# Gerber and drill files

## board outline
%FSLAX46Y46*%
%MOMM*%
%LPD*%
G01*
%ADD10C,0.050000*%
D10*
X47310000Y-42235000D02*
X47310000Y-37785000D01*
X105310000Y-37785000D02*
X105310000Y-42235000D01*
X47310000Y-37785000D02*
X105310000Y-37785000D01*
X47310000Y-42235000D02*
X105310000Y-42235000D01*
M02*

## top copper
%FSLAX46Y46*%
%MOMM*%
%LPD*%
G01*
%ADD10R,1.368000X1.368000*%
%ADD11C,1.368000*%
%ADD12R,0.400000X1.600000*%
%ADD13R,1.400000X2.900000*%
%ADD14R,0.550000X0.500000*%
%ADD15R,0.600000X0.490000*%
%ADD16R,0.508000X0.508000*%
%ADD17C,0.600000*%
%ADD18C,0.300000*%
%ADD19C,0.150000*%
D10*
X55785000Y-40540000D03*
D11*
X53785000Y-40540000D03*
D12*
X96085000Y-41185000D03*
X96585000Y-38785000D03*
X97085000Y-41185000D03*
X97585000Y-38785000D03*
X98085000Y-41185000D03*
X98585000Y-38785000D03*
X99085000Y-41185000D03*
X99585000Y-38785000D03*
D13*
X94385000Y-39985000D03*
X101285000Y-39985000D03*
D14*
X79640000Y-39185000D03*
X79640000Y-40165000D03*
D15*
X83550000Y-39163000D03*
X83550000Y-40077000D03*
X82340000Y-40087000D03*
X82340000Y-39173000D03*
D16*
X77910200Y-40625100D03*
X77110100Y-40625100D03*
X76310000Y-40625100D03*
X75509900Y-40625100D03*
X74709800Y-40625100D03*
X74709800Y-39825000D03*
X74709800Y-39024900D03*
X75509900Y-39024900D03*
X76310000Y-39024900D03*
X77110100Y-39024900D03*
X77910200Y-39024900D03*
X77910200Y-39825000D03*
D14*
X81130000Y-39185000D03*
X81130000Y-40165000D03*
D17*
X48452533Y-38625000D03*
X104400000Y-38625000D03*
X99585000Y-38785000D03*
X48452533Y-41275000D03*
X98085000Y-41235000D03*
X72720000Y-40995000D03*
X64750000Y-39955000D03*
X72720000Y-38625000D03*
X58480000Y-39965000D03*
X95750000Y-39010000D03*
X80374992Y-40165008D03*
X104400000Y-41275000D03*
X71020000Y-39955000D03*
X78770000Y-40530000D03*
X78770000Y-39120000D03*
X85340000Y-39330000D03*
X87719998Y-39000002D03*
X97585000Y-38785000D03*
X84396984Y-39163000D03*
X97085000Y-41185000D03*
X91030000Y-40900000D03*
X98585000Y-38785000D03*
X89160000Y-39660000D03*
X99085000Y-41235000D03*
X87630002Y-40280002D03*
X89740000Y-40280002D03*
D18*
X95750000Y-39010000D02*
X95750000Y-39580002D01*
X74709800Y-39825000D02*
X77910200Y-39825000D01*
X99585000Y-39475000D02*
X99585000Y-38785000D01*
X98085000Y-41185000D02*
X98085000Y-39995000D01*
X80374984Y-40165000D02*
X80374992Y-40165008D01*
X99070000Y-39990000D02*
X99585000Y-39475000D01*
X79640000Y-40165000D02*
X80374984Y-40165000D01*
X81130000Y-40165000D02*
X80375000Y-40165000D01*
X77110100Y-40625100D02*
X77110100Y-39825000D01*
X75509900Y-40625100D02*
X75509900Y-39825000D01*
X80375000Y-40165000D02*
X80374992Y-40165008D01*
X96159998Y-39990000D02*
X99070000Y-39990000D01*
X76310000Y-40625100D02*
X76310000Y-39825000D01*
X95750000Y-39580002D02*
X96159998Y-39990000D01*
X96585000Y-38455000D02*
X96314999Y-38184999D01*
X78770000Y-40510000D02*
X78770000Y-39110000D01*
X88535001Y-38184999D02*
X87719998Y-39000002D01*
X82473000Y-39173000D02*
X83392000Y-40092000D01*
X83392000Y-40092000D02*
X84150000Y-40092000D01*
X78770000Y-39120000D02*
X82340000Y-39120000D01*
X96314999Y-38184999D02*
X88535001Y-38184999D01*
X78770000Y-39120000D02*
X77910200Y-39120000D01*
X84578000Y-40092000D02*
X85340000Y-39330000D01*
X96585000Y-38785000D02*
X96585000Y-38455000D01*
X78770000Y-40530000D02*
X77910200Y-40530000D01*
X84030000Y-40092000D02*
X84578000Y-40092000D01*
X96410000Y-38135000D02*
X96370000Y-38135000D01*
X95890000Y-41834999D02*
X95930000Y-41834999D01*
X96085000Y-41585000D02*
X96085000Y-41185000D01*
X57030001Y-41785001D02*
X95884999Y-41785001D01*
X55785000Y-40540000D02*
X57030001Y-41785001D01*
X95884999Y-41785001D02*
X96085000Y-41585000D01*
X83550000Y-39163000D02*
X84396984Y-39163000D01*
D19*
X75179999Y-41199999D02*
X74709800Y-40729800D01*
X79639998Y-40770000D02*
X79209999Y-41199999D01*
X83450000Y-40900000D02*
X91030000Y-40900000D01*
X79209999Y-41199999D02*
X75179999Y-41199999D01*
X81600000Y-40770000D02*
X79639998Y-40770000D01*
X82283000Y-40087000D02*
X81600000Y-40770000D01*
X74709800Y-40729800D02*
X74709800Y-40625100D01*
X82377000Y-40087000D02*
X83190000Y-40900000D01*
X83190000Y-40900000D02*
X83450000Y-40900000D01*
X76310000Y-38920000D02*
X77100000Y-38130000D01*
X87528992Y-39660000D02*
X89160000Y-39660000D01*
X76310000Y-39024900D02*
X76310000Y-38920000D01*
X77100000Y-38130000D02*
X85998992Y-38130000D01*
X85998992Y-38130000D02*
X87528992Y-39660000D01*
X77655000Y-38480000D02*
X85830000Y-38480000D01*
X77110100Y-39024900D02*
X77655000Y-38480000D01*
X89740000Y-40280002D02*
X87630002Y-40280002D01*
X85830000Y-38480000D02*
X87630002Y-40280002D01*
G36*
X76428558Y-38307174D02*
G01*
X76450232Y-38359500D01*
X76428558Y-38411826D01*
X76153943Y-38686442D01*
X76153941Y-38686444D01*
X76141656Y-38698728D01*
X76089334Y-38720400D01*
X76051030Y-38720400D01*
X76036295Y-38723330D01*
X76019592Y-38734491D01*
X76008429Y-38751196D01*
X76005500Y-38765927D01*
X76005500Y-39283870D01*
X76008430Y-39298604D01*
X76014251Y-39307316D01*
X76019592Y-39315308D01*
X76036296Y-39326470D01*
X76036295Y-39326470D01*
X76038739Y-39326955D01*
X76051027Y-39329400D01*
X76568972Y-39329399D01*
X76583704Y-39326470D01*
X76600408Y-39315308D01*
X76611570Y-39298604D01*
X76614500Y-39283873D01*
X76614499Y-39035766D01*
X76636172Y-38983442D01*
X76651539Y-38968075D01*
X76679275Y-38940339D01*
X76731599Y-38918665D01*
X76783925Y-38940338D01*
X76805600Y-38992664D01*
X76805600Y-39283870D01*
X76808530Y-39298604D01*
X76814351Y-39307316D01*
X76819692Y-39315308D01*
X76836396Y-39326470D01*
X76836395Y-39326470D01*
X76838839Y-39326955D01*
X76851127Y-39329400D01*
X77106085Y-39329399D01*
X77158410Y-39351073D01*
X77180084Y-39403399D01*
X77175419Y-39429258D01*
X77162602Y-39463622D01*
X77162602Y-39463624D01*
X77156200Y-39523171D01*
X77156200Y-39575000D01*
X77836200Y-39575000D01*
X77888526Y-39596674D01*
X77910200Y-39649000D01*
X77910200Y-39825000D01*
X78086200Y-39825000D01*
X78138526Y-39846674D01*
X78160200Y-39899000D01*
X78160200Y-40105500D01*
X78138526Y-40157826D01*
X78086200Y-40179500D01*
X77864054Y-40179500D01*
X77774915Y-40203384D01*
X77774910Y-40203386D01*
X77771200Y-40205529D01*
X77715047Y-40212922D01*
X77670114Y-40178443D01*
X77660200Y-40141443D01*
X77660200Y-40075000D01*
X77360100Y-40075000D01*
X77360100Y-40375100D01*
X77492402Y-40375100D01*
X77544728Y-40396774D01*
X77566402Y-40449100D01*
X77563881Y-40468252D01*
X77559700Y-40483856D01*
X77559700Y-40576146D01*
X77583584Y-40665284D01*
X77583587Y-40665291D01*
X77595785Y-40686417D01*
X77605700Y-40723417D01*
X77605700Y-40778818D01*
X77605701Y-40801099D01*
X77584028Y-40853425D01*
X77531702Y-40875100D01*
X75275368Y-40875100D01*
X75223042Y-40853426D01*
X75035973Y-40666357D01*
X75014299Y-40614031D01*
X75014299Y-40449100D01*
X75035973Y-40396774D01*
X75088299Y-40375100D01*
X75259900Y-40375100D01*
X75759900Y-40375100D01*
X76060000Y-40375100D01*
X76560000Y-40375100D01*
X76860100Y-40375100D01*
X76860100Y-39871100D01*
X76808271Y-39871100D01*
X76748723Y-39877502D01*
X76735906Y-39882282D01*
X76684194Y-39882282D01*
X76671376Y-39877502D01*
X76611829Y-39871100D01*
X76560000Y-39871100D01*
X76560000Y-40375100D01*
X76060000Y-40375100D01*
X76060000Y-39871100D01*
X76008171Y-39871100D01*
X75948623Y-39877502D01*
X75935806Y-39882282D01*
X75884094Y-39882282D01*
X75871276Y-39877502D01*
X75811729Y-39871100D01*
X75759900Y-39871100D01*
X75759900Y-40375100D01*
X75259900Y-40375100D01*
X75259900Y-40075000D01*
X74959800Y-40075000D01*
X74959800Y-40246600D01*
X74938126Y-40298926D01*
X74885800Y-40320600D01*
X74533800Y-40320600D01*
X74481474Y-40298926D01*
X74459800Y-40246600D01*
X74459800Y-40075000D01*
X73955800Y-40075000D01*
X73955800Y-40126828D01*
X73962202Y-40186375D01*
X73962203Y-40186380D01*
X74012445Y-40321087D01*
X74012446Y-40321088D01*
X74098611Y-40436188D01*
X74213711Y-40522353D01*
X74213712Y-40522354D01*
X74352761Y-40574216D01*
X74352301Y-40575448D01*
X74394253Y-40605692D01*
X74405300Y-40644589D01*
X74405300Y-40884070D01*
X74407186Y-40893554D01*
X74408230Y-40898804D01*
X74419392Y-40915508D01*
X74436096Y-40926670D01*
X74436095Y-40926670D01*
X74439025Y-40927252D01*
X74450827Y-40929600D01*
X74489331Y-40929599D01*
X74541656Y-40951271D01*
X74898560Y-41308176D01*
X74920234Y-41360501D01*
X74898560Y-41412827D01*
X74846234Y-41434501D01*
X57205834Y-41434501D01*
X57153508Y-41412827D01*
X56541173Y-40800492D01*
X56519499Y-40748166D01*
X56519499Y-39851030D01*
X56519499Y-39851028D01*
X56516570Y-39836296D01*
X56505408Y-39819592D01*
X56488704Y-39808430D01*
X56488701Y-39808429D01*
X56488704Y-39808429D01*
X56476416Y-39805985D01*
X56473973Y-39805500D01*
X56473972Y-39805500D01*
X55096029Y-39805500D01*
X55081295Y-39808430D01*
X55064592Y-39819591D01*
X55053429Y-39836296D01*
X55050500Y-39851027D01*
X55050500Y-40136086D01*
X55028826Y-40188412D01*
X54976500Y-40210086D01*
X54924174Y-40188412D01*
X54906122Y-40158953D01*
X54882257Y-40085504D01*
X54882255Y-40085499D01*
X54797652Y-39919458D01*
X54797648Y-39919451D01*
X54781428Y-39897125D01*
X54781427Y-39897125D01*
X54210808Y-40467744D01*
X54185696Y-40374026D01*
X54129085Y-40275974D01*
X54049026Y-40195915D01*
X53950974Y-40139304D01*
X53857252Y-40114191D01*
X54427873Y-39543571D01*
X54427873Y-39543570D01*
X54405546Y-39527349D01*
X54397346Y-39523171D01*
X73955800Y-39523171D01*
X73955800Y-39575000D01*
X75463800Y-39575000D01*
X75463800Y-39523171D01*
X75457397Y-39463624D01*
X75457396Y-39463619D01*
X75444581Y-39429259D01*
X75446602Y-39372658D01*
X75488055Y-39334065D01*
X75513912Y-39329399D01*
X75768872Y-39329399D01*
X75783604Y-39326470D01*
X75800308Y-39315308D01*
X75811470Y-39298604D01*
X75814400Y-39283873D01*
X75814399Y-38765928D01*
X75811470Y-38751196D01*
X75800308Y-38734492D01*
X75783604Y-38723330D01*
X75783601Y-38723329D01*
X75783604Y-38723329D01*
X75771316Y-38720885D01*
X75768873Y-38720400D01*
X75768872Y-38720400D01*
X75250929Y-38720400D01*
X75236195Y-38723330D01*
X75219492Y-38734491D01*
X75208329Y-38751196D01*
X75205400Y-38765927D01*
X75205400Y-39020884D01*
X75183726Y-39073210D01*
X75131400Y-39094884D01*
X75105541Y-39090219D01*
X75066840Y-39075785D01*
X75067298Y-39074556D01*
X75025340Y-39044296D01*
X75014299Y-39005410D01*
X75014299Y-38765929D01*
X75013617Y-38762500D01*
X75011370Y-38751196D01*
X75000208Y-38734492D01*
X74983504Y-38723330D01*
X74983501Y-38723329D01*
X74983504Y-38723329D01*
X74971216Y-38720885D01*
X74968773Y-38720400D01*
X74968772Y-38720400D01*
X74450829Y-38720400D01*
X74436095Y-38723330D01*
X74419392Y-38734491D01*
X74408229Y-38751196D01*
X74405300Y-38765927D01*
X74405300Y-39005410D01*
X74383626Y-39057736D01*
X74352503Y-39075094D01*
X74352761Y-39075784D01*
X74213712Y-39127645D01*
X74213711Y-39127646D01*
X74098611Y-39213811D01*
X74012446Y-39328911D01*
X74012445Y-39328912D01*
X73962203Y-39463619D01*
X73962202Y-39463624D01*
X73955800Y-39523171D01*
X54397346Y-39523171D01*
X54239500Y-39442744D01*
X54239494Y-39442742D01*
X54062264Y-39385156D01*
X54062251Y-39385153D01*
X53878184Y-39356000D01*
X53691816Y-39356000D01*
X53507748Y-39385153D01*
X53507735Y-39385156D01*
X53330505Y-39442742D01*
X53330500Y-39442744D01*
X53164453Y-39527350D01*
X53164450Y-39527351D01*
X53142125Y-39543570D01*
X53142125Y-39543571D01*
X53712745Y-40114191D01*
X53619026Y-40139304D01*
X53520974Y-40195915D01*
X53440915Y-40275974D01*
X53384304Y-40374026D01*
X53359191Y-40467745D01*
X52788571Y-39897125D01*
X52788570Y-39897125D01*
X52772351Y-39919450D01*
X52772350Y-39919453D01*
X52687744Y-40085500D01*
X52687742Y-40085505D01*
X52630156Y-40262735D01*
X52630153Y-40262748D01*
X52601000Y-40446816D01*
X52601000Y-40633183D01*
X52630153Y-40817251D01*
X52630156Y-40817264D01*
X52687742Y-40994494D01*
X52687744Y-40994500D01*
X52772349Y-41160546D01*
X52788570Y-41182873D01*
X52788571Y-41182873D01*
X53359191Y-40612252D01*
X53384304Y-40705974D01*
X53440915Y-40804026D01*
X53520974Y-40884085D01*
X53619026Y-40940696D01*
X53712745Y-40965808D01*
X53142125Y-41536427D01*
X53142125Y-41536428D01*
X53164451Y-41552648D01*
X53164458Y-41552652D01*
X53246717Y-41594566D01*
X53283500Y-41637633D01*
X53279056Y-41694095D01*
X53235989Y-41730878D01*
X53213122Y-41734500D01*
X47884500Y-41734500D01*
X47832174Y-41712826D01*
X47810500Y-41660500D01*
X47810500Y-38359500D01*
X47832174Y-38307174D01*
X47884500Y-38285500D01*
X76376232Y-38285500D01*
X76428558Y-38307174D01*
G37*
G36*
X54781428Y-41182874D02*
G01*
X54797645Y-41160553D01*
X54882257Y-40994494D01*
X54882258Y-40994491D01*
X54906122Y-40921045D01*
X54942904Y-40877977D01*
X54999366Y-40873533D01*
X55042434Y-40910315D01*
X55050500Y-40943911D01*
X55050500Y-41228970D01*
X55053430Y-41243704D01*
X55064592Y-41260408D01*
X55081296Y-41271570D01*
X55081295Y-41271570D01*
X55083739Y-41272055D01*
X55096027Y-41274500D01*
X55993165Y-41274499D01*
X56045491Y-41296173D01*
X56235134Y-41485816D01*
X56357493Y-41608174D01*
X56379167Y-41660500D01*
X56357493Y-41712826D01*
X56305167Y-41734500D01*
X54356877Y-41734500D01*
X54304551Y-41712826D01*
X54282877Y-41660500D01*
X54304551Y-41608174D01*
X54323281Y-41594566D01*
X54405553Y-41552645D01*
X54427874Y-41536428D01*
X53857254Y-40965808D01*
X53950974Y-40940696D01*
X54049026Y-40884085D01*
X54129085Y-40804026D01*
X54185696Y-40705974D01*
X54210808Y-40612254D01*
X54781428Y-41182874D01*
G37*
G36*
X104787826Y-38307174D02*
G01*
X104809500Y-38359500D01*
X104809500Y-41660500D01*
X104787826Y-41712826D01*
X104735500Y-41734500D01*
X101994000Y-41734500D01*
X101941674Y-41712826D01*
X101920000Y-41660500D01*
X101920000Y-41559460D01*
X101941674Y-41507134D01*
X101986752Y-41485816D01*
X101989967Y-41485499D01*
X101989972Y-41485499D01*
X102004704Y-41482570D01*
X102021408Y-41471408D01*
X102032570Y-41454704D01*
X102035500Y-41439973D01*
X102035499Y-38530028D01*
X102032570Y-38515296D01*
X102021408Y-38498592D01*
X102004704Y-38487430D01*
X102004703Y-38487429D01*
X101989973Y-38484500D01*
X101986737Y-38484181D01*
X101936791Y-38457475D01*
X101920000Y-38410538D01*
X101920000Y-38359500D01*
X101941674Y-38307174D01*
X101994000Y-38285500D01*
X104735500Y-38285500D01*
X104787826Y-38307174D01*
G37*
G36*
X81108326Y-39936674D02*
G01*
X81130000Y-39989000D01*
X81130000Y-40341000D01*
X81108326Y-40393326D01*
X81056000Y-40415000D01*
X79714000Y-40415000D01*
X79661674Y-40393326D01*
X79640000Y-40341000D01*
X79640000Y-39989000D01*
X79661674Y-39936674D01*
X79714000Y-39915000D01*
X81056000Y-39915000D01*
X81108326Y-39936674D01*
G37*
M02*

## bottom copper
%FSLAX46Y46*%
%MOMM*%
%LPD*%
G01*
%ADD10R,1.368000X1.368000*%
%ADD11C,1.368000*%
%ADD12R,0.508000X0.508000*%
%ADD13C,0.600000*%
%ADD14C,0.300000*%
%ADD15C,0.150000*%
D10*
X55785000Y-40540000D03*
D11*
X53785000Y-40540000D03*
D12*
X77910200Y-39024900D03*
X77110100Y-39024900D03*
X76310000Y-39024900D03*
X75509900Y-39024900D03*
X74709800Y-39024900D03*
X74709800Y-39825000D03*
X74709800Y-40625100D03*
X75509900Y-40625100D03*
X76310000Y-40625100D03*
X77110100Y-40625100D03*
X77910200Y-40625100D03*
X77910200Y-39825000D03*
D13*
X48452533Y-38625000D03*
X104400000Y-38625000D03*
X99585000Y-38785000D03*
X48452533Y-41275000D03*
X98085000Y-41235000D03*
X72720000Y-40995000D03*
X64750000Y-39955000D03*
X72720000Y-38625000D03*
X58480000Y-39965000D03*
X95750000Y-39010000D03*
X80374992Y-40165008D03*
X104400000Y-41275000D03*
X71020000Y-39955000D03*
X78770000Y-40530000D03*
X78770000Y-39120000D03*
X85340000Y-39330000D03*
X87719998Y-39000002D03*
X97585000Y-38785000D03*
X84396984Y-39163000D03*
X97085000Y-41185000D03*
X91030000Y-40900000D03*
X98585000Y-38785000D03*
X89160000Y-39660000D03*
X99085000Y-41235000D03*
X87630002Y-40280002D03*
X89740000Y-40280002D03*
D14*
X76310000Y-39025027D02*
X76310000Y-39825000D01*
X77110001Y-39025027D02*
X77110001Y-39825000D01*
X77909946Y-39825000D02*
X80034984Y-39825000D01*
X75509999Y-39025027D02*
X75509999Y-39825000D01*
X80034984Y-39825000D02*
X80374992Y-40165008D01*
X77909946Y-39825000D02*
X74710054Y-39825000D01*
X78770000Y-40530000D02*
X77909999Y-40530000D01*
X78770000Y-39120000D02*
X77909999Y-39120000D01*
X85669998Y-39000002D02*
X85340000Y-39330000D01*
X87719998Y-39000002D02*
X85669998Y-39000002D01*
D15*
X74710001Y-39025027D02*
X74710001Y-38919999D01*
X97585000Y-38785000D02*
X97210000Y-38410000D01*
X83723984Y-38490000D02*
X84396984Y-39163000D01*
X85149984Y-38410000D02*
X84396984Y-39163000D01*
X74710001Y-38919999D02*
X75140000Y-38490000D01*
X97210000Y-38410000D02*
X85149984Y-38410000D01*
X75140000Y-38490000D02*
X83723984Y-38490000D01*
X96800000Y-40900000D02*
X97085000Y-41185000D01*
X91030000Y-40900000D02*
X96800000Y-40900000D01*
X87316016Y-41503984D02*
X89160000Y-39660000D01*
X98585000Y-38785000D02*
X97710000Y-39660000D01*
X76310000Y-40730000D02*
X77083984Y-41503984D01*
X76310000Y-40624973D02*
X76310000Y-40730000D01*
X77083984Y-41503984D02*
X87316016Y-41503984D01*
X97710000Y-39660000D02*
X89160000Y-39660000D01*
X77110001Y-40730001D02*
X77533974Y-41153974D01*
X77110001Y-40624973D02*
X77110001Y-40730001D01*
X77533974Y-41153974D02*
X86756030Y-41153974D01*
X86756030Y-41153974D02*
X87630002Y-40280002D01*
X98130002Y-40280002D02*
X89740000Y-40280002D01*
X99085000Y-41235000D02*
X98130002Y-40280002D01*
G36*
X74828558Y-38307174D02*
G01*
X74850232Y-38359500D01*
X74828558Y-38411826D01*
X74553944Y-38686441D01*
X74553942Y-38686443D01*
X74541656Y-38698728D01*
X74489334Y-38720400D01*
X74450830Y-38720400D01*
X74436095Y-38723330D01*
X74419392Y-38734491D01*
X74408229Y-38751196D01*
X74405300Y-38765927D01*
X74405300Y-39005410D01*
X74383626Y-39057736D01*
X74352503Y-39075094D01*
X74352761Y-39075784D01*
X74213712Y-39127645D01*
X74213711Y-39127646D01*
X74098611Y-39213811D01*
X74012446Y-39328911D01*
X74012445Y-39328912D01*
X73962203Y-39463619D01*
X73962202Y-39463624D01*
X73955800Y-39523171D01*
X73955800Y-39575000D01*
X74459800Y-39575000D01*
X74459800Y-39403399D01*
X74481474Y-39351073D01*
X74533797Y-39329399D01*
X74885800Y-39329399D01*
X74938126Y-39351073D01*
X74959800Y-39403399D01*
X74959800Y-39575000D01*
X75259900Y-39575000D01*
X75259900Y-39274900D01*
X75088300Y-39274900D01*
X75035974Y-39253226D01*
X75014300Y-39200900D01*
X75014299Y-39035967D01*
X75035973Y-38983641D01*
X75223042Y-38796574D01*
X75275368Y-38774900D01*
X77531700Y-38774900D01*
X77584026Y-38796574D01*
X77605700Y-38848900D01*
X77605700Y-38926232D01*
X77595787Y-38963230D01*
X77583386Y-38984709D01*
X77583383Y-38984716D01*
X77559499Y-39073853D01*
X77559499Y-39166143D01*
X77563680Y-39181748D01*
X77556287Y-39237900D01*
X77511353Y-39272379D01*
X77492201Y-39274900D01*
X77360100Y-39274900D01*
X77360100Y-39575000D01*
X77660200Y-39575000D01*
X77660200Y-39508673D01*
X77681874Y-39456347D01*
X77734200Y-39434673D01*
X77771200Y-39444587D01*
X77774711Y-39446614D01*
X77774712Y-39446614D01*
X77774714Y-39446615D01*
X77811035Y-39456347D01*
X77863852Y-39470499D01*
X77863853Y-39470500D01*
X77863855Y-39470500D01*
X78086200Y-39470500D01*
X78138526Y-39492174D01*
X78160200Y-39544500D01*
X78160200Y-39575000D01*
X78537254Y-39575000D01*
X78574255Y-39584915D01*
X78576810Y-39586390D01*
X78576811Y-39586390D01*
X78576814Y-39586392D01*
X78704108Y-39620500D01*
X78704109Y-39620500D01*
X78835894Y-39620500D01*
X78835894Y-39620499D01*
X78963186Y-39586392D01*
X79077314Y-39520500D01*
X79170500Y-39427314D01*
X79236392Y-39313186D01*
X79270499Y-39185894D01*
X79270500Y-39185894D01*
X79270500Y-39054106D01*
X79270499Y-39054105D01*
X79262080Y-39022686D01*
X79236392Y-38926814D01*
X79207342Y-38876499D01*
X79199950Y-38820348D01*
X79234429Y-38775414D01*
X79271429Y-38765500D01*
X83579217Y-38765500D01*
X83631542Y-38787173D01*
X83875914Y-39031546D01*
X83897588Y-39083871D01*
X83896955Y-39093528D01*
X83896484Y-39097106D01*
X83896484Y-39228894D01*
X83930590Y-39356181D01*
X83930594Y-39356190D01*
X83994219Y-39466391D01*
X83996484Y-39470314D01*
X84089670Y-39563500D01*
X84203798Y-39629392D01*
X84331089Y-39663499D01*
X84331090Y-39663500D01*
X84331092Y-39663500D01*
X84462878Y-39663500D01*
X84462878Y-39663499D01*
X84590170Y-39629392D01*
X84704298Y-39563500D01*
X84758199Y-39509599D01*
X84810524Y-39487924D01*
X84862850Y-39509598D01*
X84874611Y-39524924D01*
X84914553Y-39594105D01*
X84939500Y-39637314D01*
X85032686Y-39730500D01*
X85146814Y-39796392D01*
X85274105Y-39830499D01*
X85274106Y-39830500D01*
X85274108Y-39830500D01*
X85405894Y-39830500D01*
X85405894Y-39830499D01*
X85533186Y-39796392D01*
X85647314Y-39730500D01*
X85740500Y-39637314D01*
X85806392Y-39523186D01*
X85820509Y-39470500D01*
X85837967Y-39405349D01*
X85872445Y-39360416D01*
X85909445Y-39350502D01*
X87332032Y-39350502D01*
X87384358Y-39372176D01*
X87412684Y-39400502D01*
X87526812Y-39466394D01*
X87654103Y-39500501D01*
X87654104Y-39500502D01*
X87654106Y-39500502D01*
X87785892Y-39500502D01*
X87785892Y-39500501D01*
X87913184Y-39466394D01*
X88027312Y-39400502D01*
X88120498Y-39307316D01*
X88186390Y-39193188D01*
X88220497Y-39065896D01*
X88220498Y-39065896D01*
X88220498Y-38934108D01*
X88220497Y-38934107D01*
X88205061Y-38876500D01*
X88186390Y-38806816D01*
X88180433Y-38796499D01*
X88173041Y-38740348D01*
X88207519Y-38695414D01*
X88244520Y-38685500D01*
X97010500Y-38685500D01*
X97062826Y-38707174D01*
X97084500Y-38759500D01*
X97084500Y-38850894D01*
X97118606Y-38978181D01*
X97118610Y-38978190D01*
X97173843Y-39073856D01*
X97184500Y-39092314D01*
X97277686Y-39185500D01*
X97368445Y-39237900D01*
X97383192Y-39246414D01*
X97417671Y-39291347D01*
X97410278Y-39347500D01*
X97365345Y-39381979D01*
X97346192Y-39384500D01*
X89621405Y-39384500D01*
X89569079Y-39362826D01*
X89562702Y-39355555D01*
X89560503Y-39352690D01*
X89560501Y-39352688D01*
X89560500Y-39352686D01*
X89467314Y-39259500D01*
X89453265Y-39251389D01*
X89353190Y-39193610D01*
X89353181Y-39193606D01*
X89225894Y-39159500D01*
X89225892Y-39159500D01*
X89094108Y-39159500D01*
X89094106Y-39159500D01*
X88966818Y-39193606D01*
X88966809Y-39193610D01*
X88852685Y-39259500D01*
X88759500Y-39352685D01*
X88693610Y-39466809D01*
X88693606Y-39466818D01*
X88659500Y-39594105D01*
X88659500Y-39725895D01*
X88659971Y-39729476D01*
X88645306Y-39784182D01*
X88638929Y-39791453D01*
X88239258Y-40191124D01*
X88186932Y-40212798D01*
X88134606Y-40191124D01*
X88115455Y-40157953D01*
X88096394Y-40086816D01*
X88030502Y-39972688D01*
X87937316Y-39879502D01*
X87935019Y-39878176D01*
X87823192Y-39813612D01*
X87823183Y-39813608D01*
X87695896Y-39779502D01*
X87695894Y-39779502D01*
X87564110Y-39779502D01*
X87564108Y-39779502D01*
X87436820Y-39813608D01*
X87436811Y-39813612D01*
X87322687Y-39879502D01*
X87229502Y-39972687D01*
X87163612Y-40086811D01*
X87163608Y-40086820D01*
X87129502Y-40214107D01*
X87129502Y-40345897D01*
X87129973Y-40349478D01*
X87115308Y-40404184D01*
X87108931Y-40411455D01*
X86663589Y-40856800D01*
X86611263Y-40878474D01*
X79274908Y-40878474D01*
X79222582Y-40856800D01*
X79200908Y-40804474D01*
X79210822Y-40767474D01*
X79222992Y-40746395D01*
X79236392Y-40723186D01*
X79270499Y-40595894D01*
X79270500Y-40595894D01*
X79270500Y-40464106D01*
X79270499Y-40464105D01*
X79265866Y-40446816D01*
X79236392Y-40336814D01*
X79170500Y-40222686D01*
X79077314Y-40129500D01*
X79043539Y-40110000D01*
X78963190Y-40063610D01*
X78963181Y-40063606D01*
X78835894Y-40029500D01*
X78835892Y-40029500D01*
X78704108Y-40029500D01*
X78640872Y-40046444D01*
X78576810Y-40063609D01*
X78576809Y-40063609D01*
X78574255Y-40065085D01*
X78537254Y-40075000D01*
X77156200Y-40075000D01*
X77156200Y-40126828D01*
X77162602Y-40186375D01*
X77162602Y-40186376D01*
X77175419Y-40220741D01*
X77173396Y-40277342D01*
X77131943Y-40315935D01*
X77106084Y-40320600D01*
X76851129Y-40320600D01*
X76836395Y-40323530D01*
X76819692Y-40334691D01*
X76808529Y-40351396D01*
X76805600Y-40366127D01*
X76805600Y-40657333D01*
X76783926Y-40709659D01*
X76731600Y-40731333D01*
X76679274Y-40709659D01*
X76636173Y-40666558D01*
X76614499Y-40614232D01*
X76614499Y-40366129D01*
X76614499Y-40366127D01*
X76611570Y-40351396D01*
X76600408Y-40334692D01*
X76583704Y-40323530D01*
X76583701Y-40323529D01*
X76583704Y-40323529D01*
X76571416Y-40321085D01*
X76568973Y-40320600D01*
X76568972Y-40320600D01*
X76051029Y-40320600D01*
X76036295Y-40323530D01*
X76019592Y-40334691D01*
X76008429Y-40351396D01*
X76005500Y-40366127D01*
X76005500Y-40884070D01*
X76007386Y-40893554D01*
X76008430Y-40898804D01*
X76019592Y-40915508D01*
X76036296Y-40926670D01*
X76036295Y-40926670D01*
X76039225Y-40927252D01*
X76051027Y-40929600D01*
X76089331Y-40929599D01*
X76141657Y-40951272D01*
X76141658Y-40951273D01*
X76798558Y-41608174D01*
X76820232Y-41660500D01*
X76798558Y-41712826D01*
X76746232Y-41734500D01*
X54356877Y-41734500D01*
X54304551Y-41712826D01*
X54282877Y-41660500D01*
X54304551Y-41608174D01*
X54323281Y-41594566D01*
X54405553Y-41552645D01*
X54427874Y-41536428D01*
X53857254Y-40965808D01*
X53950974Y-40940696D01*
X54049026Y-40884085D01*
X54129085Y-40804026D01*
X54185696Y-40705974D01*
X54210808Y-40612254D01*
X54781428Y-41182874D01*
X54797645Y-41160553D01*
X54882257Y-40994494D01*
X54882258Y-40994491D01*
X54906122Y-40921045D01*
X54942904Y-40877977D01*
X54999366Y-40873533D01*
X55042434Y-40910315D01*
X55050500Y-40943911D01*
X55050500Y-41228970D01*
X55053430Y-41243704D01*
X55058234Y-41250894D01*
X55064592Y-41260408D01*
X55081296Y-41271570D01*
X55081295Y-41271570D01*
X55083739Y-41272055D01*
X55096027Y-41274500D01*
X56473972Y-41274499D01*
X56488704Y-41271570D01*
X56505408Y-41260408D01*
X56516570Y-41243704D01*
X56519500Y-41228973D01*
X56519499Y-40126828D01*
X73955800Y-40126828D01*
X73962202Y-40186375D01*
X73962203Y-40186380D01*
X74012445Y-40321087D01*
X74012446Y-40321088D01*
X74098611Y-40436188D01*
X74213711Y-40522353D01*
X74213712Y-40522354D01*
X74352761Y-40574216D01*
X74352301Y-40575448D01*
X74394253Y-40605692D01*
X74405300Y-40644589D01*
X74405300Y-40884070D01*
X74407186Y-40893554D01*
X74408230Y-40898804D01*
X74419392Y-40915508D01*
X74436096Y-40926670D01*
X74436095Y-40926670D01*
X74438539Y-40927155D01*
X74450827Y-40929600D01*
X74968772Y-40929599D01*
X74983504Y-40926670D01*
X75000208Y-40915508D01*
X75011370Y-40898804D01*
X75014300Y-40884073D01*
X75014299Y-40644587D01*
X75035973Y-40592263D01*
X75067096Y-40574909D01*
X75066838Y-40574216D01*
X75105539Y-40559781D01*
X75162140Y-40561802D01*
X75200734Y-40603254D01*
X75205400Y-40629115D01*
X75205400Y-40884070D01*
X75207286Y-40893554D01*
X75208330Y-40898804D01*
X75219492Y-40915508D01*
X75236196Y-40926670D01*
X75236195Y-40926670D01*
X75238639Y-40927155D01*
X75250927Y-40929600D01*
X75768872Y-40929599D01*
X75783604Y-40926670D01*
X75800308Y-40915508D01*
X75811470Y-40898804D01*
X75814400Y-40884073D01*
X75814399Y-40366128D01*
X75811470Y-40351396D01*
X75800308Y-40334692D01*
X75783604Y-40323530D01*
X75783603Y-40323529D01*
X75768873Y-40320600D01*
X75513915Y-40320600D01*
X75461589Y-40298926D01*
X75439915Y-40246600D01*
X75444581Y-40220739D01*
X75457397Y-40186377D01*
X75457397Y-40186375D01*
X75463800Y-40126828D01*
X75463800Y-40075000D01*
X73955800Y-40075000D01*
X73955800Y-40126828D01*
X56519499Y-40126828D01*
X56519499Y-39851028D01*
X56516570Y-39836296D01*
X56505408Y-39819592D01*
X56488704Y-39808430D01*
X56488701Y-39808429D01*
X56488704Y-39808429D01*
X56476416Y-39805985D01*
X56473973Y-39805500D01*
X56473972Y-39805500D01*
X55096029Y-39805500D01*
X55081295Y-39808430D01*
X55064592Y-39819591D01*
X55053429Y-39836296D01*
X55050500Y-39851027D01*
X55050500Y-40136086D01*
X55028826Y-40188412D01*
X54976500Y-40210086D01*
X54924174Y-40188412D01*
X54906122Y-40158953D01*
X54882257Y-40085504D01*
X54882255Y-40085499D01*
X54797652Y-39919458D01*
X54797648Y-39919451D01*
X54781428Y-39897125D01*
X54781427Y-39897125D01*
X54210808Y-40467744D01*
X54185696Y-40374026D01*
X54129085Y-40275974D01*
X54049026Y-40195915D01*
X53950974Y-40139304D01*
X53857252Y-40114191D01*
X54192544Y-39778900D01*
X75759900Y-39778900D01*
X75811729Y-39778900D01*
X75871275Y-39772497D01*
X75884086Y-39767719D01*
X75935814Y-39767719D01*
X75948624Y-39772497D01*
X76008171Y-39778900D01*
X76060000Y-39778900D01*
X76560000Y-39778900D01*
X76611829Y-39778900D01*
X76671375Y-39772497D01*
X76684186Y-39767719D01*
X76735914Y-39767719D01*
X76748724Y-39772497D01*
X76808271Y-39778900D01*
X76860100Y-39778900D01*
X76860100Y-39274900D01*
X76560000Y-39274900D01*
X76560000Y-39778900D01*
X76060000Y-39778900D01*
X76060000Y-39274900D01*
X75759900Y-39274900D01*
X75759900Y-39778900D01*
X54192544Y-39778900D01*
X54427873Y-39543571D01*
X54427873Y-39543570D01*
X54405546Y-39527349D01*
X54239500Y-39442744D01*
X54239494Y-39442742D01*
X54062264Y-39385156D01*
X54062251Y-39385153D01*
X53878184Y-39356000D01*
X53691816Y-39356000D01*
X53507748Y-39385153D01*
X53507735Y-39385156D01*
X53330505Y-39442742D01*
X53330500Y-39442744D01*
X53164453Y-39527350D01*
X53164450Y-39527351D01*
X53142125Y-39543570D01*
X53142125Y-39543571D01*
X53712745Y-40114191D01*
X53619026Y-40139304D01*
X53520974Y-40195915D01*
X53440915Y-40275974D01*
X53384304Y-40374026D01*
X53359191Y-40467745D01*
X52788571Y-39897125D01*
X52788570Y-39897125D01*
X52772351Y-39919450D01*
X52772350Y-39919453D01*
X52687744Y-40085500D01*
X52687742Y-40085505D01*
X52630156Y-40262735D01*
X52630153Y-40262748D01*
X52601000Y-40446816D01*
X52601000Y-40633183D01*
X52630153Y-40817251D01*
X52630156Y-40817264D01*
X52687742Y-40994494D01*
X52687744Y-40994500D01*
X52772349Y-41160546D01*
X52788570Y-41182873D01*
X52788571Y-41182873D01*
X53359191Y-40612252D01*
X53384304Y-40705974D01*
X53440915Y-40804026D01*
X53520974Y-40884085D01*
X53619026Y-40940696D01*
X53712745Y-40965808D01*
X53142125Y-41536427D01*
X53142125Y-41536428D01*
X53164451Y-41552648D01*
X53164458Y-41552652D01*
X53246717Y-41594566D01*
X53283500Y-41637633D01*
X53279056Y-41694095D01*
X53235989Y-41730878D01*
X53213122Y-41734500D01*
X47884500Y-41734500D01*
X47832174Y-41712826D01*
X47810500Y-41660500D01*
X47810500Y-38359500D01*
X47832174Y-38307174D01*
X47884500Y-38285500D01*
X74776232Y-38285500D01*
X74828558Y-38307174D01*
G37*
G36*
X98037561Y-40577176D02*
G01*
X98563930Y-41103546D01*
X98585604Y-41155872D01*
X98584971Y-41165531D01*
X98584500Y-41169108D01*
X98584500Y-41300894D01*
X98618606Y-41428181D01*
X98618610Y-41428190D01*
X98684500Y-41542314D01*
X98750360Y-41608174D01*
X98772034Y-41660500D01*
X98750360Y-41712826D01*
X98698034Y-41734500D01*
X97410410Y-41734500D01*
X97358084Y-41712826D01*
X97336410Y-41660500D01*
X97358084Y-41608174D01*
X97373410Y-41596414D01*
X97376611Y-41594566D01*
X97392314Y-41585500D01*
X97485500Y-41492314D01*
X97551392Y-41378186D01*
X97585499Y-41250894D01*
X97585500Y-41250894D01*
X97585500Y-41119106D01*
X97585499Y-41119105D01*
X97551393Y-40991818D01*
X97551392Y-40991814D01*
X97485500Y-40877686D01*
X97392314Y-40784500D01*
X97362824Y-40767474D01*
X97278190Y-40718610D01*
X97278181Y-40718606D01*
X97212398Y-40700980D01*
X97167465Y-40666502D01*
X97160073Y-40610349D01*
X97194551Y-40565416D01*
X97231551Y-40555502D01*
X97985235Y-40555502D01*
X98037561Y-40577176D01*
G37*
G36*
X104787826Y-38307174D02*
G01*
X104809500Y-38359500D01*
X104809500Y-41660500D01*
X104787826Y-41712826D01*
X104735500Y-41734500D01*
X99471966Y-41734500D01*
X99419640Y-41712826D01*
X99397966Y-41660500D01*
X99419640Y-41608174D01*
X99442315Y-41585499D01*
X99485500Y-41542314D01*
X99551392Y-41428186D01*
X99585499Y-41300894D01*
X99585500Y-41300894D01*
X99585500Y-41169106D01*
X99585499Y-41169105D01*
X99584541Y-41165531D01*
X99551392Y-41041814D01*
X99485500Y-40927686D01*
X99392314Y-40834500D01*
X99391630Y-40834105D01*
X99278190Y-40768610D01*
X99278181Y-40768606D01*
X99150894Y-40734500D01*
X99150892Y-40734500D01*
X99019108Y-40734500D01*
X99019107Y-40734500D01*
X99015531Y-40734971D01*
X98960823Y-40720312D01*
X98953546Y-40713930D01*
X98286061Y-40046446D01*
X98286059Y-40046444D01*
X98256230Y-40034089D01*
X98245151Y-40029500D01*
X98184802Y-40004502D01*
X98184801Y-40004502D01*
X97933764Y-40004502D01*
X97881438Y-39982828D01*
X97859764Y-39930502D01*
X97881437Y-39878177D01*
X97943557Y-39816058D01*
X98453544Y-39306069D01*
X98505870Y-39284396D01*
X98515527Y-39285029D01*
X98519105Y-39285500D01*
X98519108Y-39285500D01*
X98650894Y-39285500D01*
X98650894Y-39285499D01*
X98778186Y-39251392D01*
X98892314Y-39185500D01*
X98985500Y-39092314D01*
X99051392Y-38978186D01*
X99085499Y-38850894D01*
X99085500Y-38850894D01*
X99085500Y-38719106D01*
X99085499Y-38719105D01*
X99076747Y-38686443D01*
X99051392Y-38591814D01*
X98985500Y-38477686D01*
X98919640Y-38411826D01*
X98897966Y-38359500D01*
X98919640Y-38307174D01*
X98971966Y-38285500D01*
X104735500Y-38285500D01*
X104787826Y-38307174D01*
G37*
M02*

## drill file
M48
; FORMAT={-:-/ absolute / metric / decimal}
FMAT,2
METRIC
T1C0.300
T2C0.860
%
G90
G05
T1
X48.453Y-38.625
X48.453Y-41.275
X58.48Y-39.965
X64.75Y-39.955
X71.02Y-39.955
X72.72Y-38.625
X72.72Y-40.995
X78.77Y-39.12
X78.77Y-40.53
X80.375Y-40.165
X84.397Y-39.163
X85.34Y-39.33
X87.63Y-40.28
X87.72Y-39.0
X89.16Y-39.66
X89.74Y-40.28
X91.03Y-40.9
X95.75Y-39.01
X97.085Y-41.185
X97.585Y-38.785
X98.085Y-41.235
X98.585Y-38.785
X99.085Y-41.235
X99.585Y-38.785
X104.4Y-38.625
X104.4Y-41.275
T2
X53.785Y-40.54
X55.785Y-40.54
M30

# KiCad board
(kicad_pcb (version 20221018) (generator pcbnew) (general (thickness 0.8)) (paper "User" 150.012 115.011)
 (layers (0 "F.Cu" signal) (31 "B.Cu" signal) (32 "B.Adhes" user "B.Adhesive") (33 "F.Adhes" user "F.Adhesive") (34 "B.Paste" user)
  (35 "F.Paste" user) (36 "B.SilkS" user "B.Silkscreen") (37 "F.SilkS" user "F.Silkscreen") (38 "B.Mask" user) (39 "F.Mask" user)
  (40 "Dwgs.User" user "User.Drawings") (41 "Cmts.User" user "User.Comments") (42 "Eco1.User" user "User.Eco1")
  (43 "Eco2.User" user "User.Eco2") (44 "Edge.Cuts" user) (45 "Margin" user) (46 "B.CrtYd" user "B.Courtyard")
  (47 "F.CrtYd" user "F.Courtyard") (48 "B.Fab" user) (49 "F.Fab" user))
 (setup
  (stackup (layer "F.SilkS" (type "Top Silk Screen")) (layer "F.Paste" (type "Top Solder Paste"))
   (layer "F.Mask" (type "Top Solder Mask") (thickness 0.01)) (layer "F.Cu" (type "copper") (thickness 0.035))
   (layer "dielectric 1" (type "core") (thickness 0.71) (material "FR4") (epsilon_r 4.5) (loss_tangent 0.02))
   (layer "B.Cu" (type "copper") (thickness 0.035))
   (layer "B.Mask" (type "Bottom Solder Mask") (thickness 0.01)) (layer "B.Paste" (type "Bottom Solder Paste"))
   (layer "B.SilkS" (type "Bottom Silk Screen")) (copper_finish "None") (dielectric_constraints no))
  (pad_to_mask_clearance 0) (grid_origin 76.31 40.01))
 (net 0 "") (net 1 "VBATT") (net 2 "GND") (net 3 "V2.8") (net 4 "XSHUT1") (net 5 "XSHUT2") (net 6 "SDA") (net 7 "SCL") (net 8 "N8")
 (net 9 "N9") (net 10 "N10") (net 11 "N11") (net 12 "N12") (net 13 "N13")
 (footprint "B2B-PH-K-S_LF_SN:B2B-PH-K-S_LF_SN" (layer "F.Cu") (at 54.785 39.99) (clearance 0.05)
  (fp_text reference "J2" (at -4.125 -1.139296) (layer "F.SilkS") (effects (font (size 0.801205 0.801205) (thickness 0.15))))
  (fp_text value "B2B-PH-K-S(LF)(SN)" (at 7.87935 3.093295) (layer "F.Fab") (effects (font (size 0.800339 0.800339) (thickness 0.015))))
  (pad "1" thru_hole rect (at 1 0.55) (size 1.368 1.368) (drill 0.86) (layers "*.Cu" "*.Mask") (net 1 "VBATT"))
  (pad "2" thru_hole circle (at -1 0.55) (size 1.368 1.368) (drill 0.86) (layers "*.Cu" "*.Mask") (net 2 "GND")))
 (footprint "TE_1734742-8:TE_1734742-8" (layer "F.Cu") (at 97.835 39.985) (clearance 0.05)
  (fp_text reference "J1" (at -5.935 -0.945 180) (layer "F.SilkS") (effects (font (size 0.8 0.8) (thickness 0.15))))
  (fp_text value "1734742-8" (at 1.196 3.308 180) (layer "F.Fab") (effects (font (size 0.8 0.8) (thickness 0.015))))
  (pad "1" smd rect (at -1.75 1.2) (size 0.4 1.6) (layers "F.Cu" "F.Paste" "F.Mask") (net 1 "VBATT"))
  (pad "2" smd rect (at -1.25 -1.2) (size 0.4 1.6) (layers "F.Cu" "F.Paste" "F.Mask") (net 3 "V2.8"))
  (pad "3" smd rect (at -0.75 1.2) (size 0.4 1.6) (layers "F.Cu" "F.Paste" "F.Mask") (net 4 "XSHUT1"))
  (pad "4" smd rect (at -0.25 -1.2) (size 0.4 1.6) (layers "F.Cu" "F.Paste" "F.Mask") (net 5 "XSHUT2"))
  (pad "5" smd rect (at 0.25 1.2) (size 0.4 1.6) (layers "F.Cu" "F.Paste" "F.Mask") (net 2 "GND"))
  (pad "6" smd rect (at 0.75 -1.2) (size 0.4 1.6) (layers "F.Cu" "F.Paste" "F.Mask") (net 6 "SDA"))
  (pad "7" smd rect (at 1.25 1.2) (size 0.4 1.6) (layers "F.Cu" "F.Paste" "F.Mask") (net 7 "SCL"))
  (pad "8" smd rect (at 1.75 -1.2) (size 0.4 1.6) (layers "F.Cu" "F.Paste" "F.Mask") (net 2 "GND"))
  (pad "S1" smd rect (at -3.45 0) (size 1.4 2.9) (layers "F.Cu" "F.Paste" "F.Mask") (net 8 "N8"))
  (pad "S2" smd rect (at 3.45 0) (size 1.4 2.9) (layers "F.Cu" "F.Paste" "F.Mask") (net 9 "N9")))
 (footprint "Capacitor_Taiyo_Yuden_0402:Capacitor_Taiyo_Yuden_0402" (layer "F.Cu") (at 79.64 39.675 -90) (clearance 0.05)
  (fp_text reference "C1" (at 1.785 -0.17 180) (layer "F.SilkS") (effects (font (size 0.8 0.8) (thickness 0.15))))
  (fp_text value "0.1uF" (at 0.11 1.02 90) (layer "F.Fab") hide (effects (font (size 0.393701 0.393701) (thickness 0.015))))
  (pad "1" smd rect (at -0.49 0 270) (size 0.5 0.55) (layers "F.Cu" "F.Paste" "F.Mask") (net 3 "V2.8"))
  (pad "2" smd rect (at 0.49 0 270) (size 0.5 0.55) (layers "F.Cu" "F.Paste" "F.Mask") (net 2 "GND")))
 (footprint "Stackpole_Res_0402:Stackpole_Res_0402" (layer "F.Cu") (at 83.55 39.62 -90) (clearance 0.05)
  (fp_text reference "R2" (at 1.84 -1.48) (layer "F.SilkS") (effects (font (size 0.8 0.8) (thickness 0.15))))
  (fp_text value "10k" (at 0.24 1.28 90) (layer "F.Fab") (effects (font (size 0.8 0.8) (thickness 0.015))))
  (pad "1" smd rect (at -0.457 0 270) (size 0.49 0.6) (layers "F.Cu" "F.Paste" "F.Mask") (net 5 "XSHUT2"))
  (pad "2" smd rect (at 0.457 0 270) (size 0.49 0.6) (layers "F.Cu" "F.Paste" "F.Mask") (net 3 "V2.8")))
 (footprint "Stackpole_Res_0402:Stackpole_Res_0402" (layer "F.Cu") (at 82.34 39.63 90) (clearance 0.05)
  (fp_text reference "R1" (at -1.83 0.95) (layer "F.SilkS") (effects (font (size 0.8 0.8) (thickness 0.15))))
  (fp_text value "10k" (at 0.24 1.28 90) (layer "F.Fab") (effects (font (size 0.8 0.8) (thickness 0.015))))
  (pad "1" smd rect (at -0.457 0 90) (size 0.49 0.6) (layers "F.Cu" "F.Paste" "F.Mask") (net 4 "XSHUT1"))
  (pad "2" smd rect (at 0.457 0 90) (size 0.49 0.6) (layers "F.Cu" "F.Paste" "F.Mask") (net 3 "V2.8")))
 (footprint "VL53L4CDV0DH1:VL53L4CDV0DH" (layer "F.Cu") (at 76.31 39.825 -90) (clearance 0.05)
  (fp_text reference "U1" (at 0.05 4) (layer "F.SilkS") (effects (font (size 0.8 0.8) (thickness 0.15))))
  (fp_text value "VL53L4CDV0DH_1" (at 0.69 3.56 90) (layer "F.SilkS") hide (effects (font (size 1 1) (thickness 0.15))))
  (pad "1" smd rect (at 0.8001 -1.6002) (size 0.508 0.508) (layers "F.Cu" "F.Mask") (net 3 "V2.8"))
  (pad "2" smd rect (at 0.8001 -0.8001) (size 0.508 0.508) (layers "F.Cu" "F.Mask") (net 2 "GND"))
  (pad "3" smd rect (at 0.8001 0) (size 0.508 0.508) (layers "F.Cu" "F.Mask") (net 2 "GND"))
  (pad "4" smd rect (at 0.8001 0.8001) (size 0.508 0.508) (layers "F.Cu" "F.Mask") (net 2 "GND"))
  (pad "5" smd rect (at 0.8001 1.6002) (size 0.508 0.508) (layers "F.Cu" "F.Mask") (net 4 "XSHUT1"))
  (pad "6" smd rect (at 0 1.6002 270) (size 0.508 0.508) (layers "F.Cu" "F.Mask") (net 2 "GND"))
  (pad "7" smd rect (at -0.8001 1.6002) (size 0.508 0.508) (layers "F.Cu" "F.Mask") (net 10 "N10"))
  (pad "8" smd rect (at -0.8001 0.8001) (size 0.508 0.508) (layers "F.Cu" "F.Mask") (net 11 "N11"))
  (pad "9" smd rect (at -0.8001 0) (size 0.508 0.508) (layers "F.Cu" "F.Mask") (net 6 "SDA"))
  (pad "10" smd rect (at -0.8001 -0.8001) (size 0.508 0.508) (layers "F.Cu" "F.Mask") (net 7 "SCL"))
  (pad "11" smd rect (at -0.8001 -1.6002) (size 0.508 0.508) (layers "F.Cu" "F.Mask") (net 3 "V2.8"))
  (pad "12" smd rect (at 0 -1.6002 270) (size 0.508 0.508) (layers "F.Cu" "F.Mask") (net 2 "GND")))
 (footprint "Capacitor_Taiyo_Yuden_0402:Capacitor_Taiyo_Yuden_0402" (layer "F.Cu") (at 81.13 39.675 -90) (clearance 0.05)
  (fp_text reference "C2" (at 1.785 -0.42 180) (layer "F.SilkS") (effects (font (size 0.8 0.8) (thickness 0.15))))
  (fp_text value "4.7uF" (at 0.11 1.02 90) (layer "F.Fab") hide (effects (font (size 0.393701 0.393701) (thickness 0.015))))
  (pad "1" smd rect (at -0.49 0 270) (size 0.5 0.55) (layers "F.Cu" "F.Paste" "F.Mask") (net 3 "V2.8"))
  (pad "2" smd rect (at 0.49 0 270) (size 0.5 0.55) (layers "F.Cu" "F.Paste" "F.Mask") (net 2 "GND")))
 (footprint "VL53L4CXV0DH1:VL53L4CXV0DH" (layer "B.Cu") (at 76.31 39.825 -90) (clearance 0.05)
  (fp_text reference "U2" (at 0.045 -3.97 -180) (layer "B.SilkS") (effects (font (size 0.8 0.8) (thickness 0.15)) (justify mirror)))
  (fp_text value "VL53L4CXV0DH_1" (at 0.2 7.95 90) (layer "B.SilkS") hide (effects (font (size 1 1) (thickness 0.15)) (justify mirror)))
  (pad "1" smd rect (at -0.8001 -1.6002) (size 0.508 0.508) (layers "B.Cu" "B.Mask") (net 3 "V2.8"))
  (pad "2" smd rect (at -0.8001 -0.8001) (size 0.508 0.508) (layers "B.Cu" "B.Mask") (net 2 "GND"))
  (pad "3" smd rect (at -0.8001 0) (size 0.508 0.508) (layers "B.Cu" "B.Mask") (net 2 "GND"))
  (pad "4" smd rect (at -0.8001 0.8001) (size 0.508 0.508) (layers "B.Cu" "B.Mask") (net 2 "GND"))
  (pad "5" smd rect (at -0.8001 1.6002) (size 0.508 0.508) (layers "B.Cu" "B.Mask") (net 5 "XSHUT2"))
  (pad "6" smd rect (at 0 1.6002 270) (size 0.508 0.508) (layers "B.Cu" "B.Mask") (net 2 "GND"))
  (pad "7" smd rect (at 0.8001 1.6002) (size 0.508 0.508) (layers "B.Cu" "B.Mask") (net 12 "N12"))
  (pad "8" smd rect (at 0.8001 0.8001) (size 0.508 0.508) (layers "B.Cu" "B.Mask") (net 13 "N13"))
  (pad "9" smd rect (at 0.8001 0) (size 0.508 0.508) (layers "B.Cu" "B.Mask") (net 6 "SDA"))
  (pad "10" smd rect (at 0.8001 -0.8001) (size 0.508 0.508) (layers "B.Cu" "B.Mask") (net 7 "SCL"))
  (pad "11" smd rect (at 0.8001 -1.6002) (size 0.508 0.508) (layers "B.Cu" "B.Mask") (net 3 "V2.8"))
  (pad "12" smd rect (at 0 -1.6002 270) (size 0.508 0.508) (layers "B.Cu" "B.Mask") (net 2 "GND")))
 (gr_line (start 47.31 42.235) (end 47.31 37.785) (stroke (width 0.05) (type solid)) (layer "Edge.Cuts"))
 (gr_line (start 105.31 37.785) (end 105.31 42.235) (stroke (width 0.05) (type solid)) (layer "Edge.Cuts"))
 (gr_line (start 47.31 37.785) (end 105.31 37.785) (stroke (width 0.05) (type solid)) (layer "Edge.Cuts"))
 (gr_line (start 47.31 42.235) (end 105.31 42.235) (stroke (width 0.05) (type solid)) (layer "Edge.Cuts"))
 (segment (start 95.75 39.01) (end 95.75 39.580002) (width 0.3) (layer "F.Cu") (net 2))
 (segment (start 74.7098 39.825) (end 77.9102 39.825) (width 0.3) (layer "F.Cu") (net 2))
 (segment (start 99.585 39.475) (end 99.585 38.785) (width 0.3) (layer "F.Cu") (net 2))
 (segment (start 98.085 41.185) (end 98.085 39.995) (width 0.3) (layer "F.Cu") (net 2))
 (segment (start 80.374984 40.165) (end 80.374992 40.165008) (width 0.3) (layer "F.Cu") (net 2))
 (segment (start 99.07 39.99) (end 99.585 39.475) (width 0.3) (layer "F.Cu") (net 2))
 (segment (start 79.64 40.165) (end 80.374984 40.165) (width 0.3) (layer "F.Cu") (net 2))
 (segment (start 81.13 40.165) (end 80.375 40.165) (width 0.3) (layer "F.Cu") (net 2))
 (segment (start 77.1101 40.6251) (end 77.1101 39.825) (width 0.3) (layer "F.Cu") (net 2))
 (segment (start 75.5099 40.6251) (end 75.5099 39.825) (width 0.3) (layer "F.Cu") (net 2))
 (segment (start 80.375 40.165) (end 80.374992 40.165008) (width 0.3) (layer "F.Cu") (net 2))
 (segment (start 96.159998 39.99) (end 99.07 39.99) (width 0.3) (layer "F.Cu") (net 2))
 (segment (start 76.31 40.6251) (end 76.31 39.825) (width 0.3) (layer "F.Cu") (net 2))
 (segment (start 95.75 39.580002) (end 96.159998 39.99) (width 0.3) (layer "F.Cu") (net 2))
 (via (at 48.452533 38.625) (size 0.6) (drill 0.3) (layers "F.Cu" "B.Cu") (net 2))
 (via (at 104.4 38.625) (size 0.6) (drill 0.3) (layers "F.Cu" "B.Cu") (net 2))
 (via (at 99.585 38.785) (size 0.6) (drill 0.3) (layers "F.Cu" "B.Cu") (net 2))
 (via (at 48.452533 41.275) (size 0.6) (drill 0.3) (layers "F.Cu" "B.Cu") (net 2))
 (via (at 98.085 41.235) (size 0.6) (drill 0.3) (layers "F.Cu" "B.Cu") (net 2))
 (via (at 72.72 40.995) (size 0.6) (drill 0.3) (layers "F.Cu" "B.Cu") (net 2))
 (via (at 64.75 39.955) (size 0.6) (drill 0.3) (layers "F.Cu" "B.Cu") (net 2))
 (via (at 72.72 38.625) (size 0.6) (drill 0.3) (layers "F.Cu" "B.Cu") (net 2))
 (via (at 58.48 39.965) (size 0.6) (drill 0.3) (layers "F.Cu" "B.Cu") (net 2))
 (via (at 95.75 39.01) (size 0.6) (drill 0.3) (layers "F.Cu" "B.Cu") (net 2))
 (via (at 80.374992 40.165008) (size 0.6) (drill 0.3) (layers "F.Cu" "B.Cu") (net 2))
 (via (at 104.4 41.275) (size 0.6) (drill 0.3) (layers "F.Cu" "B.Cu") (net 2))
 (via (at 71.02 39.955) (size 0.6) (drill 0.3) (layers "F.Cu" "B.Cu") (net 2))
 (segment (start 76.31 39.025027) (end 76.31 39.825) (width 0.3) (layer "B.Cu") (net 2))
 (segment (start 77.110001 39.025027) (end 77.110001 39.825) (width 0.3) (layer "B.Cu") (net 2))
 (segment (start 77.909946 39.825) (end 80.034984 39.825) (width 0.3) (layer "B.Cu") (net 2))
 (segment (start 75.509999 39.025027) (end 75.509999 39.825) (width 0.3) (layer "B.Cu") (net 2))
 (segment (start 80.034984 39.825) (end 80.374992 40.165008) (width 0.3) (layer "B.Cu") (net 2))
 (segment (start 77.909946 39.825) (end 74.710054 39.825) (width 0.3) (layer "B.Cu") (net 2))
 (segment (start 96.585 38.455) (end 96.314999 38.184999) (width 0.3) (layer "F.Cu") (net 3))
 (segment (start 78.77 40.51) (end 78.77 39.11) (width 0.3) (layer "F.Cu") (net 3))
 (segment (start 88.535001 38.184999) (end 87.719998 39.000002) (width 0.3) (layer "F.Cu") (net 3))
 (segment (start 82.473 39.173) (end 83.392 40.092) (width 0.3) (layer "F.Cu") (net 3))
 (segment (start 83.392 40.092) (end 84.15 40.092) (width 0.3) (layer "F.Cu") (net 3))
 (segment (start 78.77 39.12) (end 82.34 39.12) (width 0.3) (layer "F.Cu") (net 3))
 (segment (start 96.314999 38.184999) (end 88.535001 38.184999) (width 0.3) (layer "F.Cu") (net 3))
 (segment (start 78.77 39.12) (end 77.9102 39.12) (width 0.3) (layer "F.Cu") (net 3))
 (segment (start 84.578 40.092) (end 85.34 39.33) (width 0.3) (layer "F.Cu") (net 3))
 (segment (start 96.585 38.785) (end 96.585 38.455) (width 0.3) (layer "F.Cu") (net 3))
 (segment (start 78.77 40.53) (end 77.9102 40.53) (width 0.3) (layer "F.Cu") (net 3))
 (segment (start 84.03 40.092) (end 84.578 40.092) (width 0.3) (layer "F.Cu") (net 3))
 (segment (start 96.41 38.135) (end 96.37 38.135) (width 0.3) (layer "F.Cu") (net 3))
 (via (at 78.77 40.53) (size 0.6) (drill 0.3) (layers "F.Cu" "B.Cu") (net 3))
 (via (at 78.77 39.12) (size 0.6) (drill 0.3) (layers "F.Cu" "B.Cu") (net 3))
 (via (at 85.34 39.33) (size 0.6) (drill 0.3) (layers "F.Cu" "B.Cu") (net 3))
 (via (at 87.719998 39.000002) (size 0.6) (drill 0.3) (layers "F.Cu" "B.Cu") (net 3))
 (segment (start 78.77 40.53) (end 77.909999 40.53) (width 0.3) (layer "B.Cu") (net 3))
 (segment (start 78.77 39.12) (end 77.909999 39.12) (width 0.3) (layer "B.Cu") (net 3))
 (segment (start 85.669998 39.000002) (end 85.34 39.33) (width 0.3) (layer "B.Cu") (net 3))
 (segment (start 87.719998 39.000002) (end 85.669998 39.000002) (width 0.3) (layer "B.Cu") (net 3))
 (segment (start 95.89 41.834999) (end 95.93 41.834999) (width 0.3) (layer "F.Cu") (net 1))
 (segment (start 96.085 41.585) (end 96.085 41.185) (width 0.3) (layer "F.Cu") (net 1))
 (segment (start 57.030001 41.785001) (end 95.884999 41.785001) (width 0.3) (layer "F.Cu") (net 1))
 (segment (start 55.785 40.54) (end 57.030001 41.785001) (width 0.3) (layer "F.Cu") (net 1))
 (segment (start 95.884999 41.785001) (end 96.085 41.585) (width 0.3) (layer "F.Cu") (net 1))
 (segment (start 83.55 39.163) (end 84.396984 39.163) (width 0.3) (layer "F.Cu") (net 5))
 (via (at 97.585 38.785) (size 0.6) (drill 0.3) (layers "F.Cu" "B.Cu") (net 5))
 (via (at 84.396984 39.163) (size 0.6) (drill 0.3) (layers "F.Cu" "B.Cu") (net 5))
 (segment (start 74.710001 39.025027) (end 74.710001 38.919999) (width 0.15) (layer "B.Cu") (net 5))
 (segment (start 97.585 38.785) (end 97.21 38.41) (width 0.15) (layer "B.Cu") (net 5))
 (segment (start 83.723984 38.49) (end 84.396984 39.163) (width 0.15) (layer "B.Cu") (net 5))
 (segment (start 85.149984 38.41) (end 84.396984 39.163) (width 0.15) (layer "B.Cu") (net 5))
 (segment (start 74.710001 38.919999) (end 75.14 38.49) (width 0.15) (layer "B.Cu") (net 5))
 (segment (start 97.21 38.41) (end 85.149984 38.41) (width 0.15) (layer "B.Cu") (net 5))
 (segment (start 75.14 38.49) (end 83.723984 38.49) (width 0.15) (layer "B.Cu") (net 5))
 (segment (start 75.179999 41.199999) (end 74.7098 40.7298) (width 0.15) (layer "F.Cu") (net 4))
 (segment (start 79.639998 40.77) (end 79.209999 41.199999) (width 0.15) (layer "F.Cu") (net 4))
 (segment (start 83.45 40.9) (end 91.03 40.9) (width 0.15) (layer "F.Cu") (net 4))
 (segment (start 79.209999 41.199999) (end 75.179999 41.199999) (width 0.15) (layer "F.Cu") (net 4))
 (segment (start 81.6 40.77) (end 79.639998 40.77) (width 0.15) (layer "F.Cu") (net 4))
 (segment (start 82.283 40.087) (end 81.6 40.77) (width 0.15) (layer "F.Cu") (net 4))
 (segment (start 74.7098 40.7298) (end 74.7098 40.6251) (width 0.15) (layer "F.Cu") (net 4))
 (segment (start 82.377 40.087) (end 83.19 40.9) (width 0.15) (layer "F.Cu") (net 4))
 (segment (start 83.19 40.9) (end 83.45 40.9) (width 0.15) (layer "F.Cu") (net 4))
 (via (at 97.085 41.185) (size 0.6) (drill 0.3) (layers "F.Cu" "B.Cu") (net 4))
 (via (at 91.03 40.9) (size 0.6) (drill 0.3) (layers "F.Cu" "B.Cu") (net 4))
 (segment (start 96.8 40.9) (end 97.085 41.185) (width 0.15) (layer "B.Cu") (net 4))
 (segment (start 91.03 40.9) (end 96.8 40.9) (width 0.15) (layer "B.Cu") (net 4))
 (segment (start 76.31 38.92) (end 77.1 38.13) (width 0.15) (layer "F.Cu") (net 6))
 (segment (start 87.528992 39.66) (end 89.16 39.66) (width 0.15) (layer "F.Cu") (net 6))
 (segment (start 76.31 39.0249) (end 76.31 38.92) (width 0.15) (layer "F.Cu") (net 6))
 (segment (start 77.1 38.13) (end 85.998992 38.13) (width 0.15) (layer "F.Cu") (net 6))
 (segment (start 85.998992 38.13) (end 87.528992 39.66) (width 0.15) (layer "F.Cu") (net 6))
 (via (at 98.585 38.785) (size 0.6) (drill 0.3) (layers "F.Cu" "B.Cu") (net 6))
 (via (at 89.16 39.66) (size 0.6) (drill 0.3) (layers "F.Cu" "B.Cu") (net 6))
 (segment (start 87.316016 41.503984) (end 89.16 39.66) (width 0.15) (layer "B.Cu") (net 6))
 (segment (start 98.585 38.785) (end 97.71 39.66) (width 0.15) (layer "B.Cu") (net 6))
 (segment (start 76.31 40.73) (end 77.083984 41.503984) (width 0.15) (layer "B.Cu") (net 6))
 (segment (start 76.31 40.624973) (end 76.31 40.73) (width 0.15) (layer "B.Cu") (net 6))
 (segment (start 77.083984 41.503984) (end 87.316016 41.503984) (width 0.15) (layer "B.Cu") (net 6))
 (segment (start 97.71 39.66) (end 89.16 39.66) (width 0.15) (layer "B.Cu") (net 6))
 (segment (start 77.655 38.48) (end 85.83 38.48) (width 0.15) (layer "F.Cu") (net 7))
 (segment (start 77.1101 39.0249) (end 77.655 38.48) (width 0.15) (layer "F.Cu") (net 7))
 (segment (start 89.74 40.280002) (end 87.630002 40.280002) (width 0.15) (layer "F.Cu") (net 7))
 (segment (start 85.83 38.48) (end 87.630002 40.280002) (width 0.15) (layer "F.Cu") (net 7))
 (via (at 99.085 41.235) (size 0.6) (drill 0.3) (layers "F.Cu" "B.Cu") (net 7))
 (via (at 87.630002 40.280002) (size 0.6) (drill 0.3) (layers "F.Cu" "B.Cu") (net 7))
 (via (at 89.74 40.280002) (size 0.6) (drill 0.3) (layers "F.Cu" "B.Cu") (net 7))
 (segment (start 77.110001 40.730001) (end 77.533974 41.153974) (width 0.15) (layer "B.Cu") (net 7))
 (segment (start 77.110001 40.624973) (end 77.110001 40.730001) (width 0.15) (layer "B.Cu") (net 7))
 (segment (start 77.533974 41.153974) (end 86.75603 41.153974) (width 0.15) (layer "B.Cu") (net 7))
 (segment (start 86.75603 41.153974) (end 87.630002 40.280002) (width 0.15) (layer "B.Cu") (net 7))
 (segment (start 98.130002 40.280002) (end 89.74 40.280002) (width 0.15) (layer "B.Cu") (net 7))
 (segment (start 99.085 41.235) (end 98.130002 40.280002) (width 0.15) (layer "B.Cu") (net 7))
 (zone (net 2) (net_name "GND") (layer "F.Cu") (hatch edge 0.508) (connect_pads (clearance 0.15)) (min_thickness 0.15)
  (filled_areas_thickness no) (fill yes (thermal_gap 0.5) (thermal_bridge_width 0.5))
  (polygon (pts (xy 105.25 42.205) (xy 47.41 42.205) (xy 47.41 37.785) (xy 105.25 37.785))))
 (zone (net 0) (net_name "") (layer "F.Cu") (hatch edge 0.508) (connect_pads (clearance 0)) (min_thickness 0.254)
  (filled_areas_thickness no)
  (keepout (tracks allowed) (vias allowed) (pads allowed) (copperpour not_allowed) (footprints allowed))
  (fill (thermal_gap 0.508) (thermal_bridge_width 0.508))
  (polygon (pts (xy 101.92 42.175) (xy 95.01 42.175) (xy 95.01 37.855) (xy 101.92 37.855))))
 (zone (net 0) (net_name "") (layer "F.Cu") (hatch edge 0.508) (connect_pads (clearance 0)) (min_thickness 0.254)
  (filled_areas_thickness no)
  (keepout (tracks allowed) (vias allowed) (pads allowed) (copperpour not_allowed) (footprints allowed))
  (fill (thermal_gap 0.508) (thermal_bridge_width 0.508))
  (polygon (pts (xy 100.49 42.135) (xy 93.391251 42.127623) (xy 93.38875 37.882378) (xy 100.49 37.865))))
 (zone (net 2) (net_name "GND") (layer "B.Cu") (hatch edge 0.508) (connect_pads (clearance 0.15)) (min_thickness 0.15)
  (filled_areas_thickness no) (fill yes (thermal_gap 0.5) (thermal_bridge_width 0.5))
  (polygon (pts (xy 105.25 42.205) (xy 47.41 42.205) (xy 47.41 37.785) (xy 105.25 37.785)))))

